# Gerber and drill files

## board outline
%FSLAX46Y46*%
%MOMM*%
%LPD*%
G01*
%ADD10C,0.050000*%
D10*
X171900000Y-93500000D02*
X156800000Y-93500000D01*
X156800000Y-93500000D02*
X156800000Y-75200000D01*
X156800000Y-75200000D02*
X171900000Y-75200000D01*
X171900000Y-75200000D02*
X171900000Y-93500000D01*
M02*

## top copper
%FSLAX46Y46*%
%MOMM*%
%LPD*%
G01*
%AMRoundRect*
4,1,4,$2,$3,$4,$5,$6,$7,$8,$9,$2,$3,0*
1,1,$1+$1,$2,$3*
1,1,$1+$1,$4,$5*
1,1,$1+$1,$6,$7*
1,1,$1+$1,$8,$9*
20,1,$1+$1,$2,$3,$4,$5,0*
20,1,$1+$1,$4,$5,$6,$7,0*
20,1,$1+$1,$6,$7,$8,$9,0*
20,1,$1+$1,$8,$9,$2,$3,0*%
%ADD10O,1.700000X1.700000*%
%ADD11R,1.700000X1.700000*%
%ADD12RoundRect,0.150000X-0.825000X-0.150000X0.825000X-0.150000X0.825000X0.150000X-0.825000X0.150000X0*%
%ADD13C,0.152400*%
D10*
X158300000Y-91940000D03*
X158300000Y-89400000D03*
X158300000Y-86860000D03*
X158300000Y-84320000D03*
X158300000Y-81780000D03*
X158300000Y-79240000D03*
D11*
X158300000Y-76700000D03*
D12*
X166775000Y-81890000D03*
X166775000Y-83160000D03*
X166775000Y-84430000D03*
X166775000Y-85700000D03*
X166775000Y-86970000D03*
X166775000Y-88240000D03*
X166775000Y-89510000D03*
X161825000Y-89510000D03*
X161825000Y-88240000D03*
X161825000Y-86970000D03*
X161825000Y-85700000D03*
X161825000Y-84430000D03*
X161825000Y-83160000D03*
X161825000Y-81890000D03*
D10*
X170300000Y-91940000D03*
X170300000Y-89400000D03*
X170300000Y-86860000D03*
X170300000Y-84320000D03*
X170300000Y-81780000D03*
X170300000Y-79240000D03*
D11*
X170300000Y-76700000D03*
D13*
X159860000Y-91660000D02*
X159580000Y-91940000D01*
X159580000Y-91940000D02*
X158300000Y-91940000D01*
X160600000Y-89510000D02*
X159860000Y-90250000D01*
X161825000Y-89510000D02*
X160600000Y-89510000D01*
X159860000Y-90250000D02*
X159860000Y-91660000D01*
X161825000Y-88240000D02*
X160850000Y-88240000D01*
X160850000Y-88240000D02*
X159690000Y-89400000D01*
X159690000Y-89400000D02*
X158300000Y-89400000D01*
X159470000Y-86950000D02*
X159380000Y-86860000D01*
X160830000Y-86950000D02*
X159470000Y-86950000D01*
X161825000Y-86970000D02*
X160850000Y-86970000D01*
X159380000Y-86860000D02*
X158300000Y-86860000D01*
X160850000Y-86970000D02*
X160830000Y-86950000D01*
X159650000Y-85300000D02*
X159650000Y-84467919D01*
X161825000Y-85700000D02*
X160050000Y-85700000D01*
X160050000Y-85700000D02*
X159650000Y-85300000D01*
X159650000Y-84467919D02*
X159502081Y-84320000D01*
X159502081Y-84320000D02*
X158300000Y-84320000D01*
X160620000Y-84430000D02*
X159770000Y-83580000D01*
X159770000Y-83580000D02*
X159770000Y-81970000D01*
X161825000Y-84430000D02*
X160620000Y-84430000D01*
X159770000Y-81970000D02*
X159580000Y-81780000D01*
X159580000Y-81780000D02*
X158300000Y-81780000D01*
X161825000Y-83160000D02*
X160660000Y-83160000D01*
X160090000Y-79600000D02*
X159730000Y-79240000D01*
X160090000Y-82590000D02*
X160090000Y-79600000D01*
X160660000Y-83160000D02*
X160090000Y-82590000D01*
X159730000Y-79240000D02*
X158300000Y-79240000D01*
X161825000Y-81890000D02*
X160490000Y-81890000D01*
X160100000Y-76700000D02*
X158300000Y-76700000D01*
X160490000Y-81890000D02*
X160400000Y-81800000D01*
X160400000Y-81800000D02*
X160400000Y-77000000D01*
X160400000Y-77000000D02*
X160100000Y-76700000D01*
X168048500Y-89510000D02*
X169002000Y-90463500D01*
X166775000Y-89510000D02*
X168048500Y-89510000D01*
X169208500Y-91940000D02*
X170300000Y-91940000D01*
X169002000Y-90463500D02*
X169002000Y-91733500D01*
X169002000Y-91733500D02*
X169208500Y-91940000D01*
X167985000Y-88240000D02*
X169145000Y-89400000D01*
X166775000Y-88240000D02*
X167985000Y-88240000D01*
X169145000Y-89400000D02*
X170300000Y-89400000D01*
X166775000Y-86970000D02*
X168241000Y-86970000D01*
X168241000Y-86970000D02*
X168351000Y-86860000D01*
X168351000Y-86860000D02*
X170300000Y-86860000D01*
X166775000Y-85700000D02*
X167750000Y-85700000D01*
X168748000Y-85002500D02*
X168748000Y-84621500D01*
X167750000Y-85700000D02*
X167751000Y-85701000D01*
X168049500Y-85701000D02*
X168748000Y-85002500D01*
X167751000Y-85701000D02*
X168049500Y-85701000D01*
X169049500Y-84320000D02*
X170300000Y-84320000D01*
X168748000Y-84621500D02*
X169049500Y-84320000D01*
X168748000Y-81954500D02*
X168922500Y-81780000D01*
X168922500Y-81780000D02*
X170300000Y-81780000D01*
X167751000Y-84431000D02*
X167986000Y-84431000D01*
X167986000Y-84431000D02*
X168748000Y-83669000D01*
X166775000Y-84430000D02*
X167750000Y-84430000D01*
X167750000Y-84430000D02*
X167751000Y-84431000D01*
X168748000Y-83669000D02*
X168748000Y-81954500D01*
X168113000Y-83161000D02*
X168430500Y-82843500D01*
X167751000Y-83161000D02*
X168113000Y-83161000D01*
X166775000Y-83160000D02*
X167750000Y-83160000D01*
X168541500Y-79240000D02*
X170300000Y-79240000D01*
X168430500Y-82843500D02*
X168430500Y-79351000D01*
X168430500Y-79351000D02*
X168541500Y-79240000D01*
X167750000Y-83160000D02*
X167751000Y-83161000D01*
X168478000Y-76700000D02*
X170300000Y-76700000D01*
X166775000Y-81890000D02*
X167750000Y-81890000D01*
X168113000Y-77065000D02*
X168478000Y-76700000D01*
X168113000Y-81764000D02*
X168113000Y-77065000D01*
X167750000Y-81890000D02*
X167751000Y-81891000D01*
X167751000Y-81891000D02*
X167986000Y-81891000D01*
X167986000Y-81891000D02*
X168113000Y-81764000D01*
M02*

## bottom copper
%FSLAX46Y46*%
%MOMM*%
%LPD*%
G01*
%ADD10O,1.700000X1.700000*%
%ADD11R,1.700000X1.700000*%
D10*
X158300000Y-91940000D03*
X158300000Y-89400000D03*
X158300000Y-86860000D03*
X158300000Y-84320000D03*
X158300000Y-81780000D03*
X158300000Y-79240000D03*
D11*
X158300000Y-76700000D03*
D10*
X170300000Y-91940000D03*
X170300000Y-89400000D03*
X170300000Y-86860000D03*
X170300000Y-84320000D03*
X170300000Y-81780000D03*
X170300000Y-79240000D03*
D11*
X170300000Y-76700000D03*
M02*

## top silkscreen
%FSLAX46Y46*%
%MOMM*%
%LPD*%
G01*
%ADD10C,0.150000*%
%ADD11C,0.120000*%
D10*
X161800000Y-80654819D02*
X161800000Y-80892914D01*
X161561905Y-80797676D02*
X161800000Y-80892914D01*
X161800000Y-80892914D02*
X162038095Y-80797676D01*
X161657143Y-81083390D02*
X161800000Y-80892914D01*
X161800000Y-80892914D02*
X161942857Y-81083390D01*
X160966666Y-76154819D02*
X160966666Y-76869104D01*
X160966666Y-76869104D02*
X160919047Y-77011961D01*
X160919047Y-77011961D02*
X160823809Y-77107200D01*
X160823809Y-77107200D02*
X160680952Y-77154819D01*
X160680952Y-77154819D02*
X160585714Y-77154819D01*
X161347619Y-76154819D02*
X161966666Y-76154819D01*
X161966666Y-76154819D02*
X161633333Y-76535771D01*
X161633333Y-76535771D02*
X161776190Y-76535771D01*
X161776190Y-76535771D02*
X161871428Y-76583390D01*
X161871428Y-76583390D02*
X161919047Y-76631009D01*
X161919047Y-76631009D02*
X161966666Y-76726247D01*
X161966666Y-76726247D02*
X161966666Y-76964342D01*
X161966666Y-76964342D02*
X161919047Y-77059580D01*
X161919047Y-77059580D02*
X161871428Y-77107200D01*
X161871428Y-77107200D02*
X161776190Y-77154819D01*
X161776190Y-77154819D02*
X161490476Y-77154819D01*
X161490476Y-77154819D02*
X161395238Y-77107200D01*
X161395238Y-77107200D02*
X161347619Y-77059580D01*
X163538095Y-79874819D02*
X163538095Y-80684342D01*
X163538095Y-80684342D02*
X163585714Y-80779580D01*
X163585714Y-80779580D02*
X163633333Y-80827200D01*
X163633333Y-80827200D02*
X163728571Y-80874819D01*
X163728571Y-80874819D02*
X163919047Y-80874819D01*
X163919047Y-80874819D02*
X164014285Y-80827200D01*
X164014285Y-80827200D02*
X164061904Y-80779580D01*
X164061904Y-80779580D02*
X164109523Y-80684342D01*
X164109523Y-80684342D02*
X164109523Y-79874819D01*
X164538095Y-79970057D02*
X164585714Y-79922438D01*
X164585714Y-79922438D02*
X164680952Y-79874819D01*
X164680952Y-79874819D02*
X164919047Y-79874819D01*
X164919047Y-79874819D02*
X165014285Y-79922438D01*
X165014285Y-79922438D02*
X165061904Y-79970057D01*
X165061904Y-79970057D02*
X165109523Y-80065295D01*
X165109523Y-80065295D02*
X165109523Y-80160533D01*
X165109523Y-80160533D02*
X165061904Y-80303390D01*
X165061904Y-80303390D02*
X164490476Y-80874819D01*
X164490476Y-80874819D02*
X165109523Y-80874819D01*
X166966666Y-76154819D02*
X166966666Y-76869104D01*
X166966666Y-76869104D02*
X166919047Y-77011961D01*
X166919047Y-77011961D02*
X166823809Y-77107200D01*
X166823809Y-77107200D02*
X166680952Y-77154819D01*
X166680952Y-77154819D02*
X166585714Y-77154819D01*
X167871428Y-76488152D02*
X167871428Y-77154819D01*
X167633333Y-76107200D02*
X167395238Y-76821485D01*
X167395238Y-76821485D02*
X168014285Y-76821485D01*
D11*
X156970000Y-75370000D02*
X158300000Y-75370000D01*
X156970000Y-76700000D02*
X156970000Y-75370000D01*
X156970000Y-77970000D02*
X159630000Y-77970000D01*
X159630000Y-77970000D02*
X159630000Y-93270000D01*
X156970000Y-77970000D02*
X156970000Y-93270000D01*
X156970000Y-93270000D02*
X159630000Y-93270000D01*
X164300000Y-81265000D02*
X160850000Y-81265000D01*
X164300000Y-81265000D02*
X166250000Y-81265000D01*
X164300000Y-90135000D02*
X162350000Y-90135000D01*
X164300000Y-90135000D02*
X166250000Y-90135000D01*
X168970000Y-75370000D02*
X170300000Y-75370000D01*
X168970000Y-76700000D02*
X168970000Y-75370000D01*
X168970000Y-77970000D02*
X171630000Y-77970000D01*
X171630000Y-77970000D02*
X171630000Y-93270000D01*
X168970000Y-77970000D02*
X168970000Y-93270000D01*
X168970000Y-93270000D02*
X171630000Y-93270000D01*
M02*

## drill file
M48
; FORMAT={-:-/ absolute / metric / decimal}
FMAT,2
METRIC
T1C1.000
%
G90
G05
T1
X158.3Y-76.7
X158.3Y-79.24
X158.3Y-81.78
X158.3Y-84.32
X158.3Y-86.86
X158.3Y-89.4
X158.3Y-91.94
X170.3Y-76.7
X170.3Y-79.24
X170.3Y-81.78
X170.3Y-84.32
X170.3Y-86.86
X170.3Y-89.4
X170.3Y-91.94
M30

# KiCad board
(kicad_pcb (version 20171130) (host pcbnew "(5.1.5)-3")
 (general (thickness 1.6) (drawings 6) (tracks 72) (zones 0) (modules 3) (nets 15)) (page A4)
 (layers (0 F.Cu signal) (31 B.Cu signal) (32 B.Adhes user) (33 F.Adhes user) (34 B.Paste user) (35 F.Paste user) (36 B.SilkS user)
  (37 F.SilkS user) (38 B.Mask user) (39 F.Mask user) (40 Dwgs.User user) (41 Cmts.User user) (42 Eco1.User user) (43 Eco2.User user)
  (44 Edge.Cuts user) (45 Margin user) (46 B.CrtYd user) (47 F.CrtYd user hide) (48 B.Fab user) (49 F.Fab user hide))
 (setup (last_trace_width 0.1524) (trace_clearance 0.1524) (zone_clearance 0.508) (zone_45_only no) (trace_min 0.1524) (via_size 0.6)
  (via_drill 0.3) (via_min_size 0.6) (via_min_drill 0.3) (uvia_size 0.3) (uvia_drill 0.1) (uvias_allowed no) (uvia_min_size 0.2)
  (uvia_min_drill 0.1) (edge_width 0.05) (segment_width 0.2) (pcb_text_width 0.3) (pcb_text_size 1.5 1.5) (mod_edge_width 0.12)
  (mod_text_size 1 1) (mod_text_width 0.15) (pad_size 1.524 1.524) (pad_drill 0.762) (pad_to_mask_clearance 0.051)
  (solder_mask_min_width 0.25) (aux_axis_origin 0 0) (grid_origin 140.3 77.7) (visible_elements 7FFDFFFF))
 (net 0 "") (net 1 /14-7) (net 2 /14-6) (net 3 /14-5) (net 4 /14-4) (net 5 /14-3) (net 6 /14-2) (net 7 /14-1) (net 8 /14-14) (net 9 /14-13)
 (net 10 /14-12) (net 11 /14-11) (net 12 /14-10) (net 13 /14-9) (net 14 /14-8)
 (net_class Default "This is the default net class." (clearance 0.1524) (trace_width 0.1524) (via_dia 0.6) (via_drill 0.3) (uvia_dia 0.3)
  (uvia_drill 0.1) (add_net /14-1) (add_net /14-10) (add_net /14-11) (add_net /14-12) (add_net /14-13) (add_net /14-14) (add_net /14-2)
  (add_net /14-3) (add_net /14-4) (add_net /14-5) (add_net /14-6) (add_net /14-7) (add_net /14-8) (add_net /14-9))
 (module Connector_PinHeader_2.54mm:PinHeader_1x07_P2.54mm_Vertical (layer F.Cu) (at 158.3 76.7)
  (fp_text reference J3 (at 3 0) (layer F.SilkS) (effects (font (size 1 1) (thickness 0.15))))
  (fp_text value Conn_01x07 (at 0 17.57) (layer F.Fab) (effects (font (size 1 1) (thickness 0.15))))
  (fp_line (start -1.33 -1.33) (end 0 -1.33) (layer F.SilkS) (width 0.12))
  (fp_line (start -1.33 0) (end -1.33 -1.33) (layer F.SilkS) (width 0.12))
  (fp_line (start -1.33 1.27) (end 1.33 1.27) (layer F.SilkS) (width 0.12))
  (fp_line (start 1.33 1.27) (end 1.33 16.57) (layer F.SilkS) (width 0.12))
  (fp_line (start -1.33 1.27) (end -1.33 16.57) (layer F.SilkS) (width 0.12))
  (fp_line (start -1.33 16.57) (end 1.33 16.57) (layer F.SilkS) (width 0.12))
  (pad 7 thru_hole oval (at 0 15.24) (size 1.7 1.7) (drill 1) (layers *.Cu *.Mask) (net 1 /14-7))
  (pad 6 thru_hole oval (at 0 12.7) (size 1.7 1.7) (drill 1) (layers *.Cu *.Mask) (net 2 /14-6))
  (pad 5 thru_hole oval (at 0 10.16) (size 1.7 1.7) (drill 1) (layers *.Cu *.Mask) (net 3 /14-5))
  (pad 4 thru_hole oval (at 0 7.62) (size 1.7 1.7) (drill 1) (layers *.Cu *.Mask) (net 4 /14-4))
  (pad 3 thru_hole oval (at 0 5.08) (size 1.7 1.7) (drill 1) (layers *.Cu *.Mask) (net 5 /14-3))
  (pad 2 thru_hole oval (at 0 2.54) (size 1.7 1.7) (drill 1) (layers *.Cu *.Mask) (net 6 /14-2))
  (pad 1 thru_hole rect (at 0 0) (size 1.7 1.7) (drill 1) (layers *.Cu *.Mask) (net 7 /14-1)))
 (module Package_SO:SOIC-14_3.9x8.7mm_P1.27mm (layer F.Cu) (at 164.3 85.7)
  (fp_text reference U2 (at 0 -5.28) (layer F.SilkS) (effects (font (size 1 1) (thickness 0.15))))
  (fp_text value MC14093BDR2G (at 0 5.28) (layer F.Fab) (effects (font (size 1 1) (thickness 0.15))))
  (fp_line (start 0 -4.435) (end -3.45 -4.435) (layer F.SilkS) (width 0.12))
  (fp_line (start 0 -4.435) (end 1.95 -4.435) (layer F.SilkS) (width 0.12))
  (fp_line (start 0 4.435) (end -1.95 4.435) (layer F.SilkS) (width 0.12))
  (fp_line (start 0 4.435) (end 1.95 4.435) (layer F.SilkS) (width 0.12))
  (pad 14 smd roundrect (at 2.475 -3.81) (size 1.95 0.6) (layers F.Cu F.Paste F.Mask) (roundrect_rratio 0.25) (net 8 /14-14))
  (pad 13 smd roundrect (at 2.475 -2.54) (size 1.95 0.6) (layers F.Cu F.Paste F.Mask) (roundrect_rratio 0.25) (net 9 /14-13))
  (pad 12 smd roundrect (at 2.475 -1.27) (size 1.95 0.6) (layers F.Cu F.Paste F.Mask) (roundrect_rratio 0.25) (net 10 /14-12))
  (pad 11 smd roundrect (at 2.475 0) (size 1.95 0.6) (layers F.Cu F.Paste F.Mask) (roundrect_rratio 0.25) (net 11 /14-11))
  (pad 10 smd roundrect (at 2.475 1.27) (size 1.95 0.6) (layers F.Cu F.Paste F.Mask) (roundrect_rratio 0.25) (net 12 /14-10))
  (pad 9 smd roundrect (at 2.475 2.54) (size 1.95 0.6) (layers F.Cu F.Paste F.Mask) (roundrect_rratio 0.25) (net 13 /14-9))
  (pad 8 smd roundrect (at 2.475 3.81) (size 1.95 0.6) (layers F.Cu F.Paste F.Mask) (roundrect_rratio 0.25) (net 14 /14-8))
  (pad 7 smd roundrect (at -2.475 3.81) (size 1.95 0.6) (layers F.Cu F.Paste F.Mask) (roundrect_rratio 0.25) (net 1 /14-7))
  (pad 6 smd roundrect (at -2.475 2.54) (size 1.95 0.6) (layers F.Cu F.Paste F.Mask) (roundrect_rratio 0.25) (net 2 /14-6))
  (pad 5 smd roundrect (at -2.475 1.27) (size 1.95 0.6) (layers F.Cu F.Paste F.Mask) (roundrect_rratio 0.25) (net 3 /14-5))
  (pad 4 smd roundrect (at -2.475 0) (size 1.95 0.6) (layers F.Cu F.Paste F.Mask) (roundrect_rratio 0.25) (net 4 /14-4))
  (pad 3 smd roundrect (at -2.475 -1.27) (size 1.95 0.6) (layers F.Cu F.Paste F.Mask) (roundrect_rratio 0.25) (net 5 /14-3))
  (pad 2 smd roundrect (at -2.475 -2.54) (size 1.95 0.6) (layers F.Cu F.Paste F.Mask) (roundrect_rratio 0.25) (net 6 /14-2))
  (pad 1 smd roundrect (at -2.475 -3.81) (size 1.95 0.6) (layers F.Cu F.Paste F.Mask) (roundrect_rratio 0.25) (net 7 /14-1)))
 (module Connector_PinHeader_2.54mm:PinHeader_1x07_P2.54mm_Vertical (layer F.Cu) (at 170.3 76.7)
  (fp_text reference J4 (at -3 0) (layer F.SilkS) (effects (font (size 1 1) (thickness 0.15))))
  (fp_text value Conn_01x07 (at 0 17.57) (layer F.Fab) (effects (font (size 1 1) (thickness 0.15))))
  (fp_line (start -1.33 -1.33) (end 0 -1.33) (layer F.SilkS) (width 0.12))
  (fp_line (start -1.33 0) (end -1.33 -1.33) (layer F.SilkS) (width 0.12))
  (fp_line (start -1.33 1.27) (end 1.33 1.27) (layer F.SilkS) (width 0.12))
  (fp_line (start 1.33 1.27) (end 1.33 16.57) (layer F.SilkS) (width 0.12))
  (fp_line (start -1.33 1.27) (end -1.33 16.57) (layer F.SilkS) (width 0.12))
  (fp_line (start -1.33 16.57) (end 1.33 16.57) (layer F.SilkS) (width 0.12))
  (pad 7 thru_hole oval (at 0 15.24) (size 1.7 1.7) (drill 1) (layers *.Cu *.Mask) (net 14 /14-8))
  (pad 6 thru_hole oval (at 0 12.7) (size 1.7 1.7) (drill 1) (layers *.Cu *.Mask) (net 13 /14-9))
  (pad 5 thru_hole oval (at 0 10.16) (size 1.7 1.7) (drill 1) (layers *.Cu *.Mask) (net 12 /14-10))
  (pad 4 thru_hole oval (at 0 7.62) (size 1.7 1.7) (drill 1) (layers *.Cu *.Mask) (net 11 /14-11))
  (pad 3 thru_hole oval (at 0 5.08) (size 1.7 1.7) (drill 1) (layers *.Cu *.Mask) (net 10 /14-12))
  (pad 2 thru_hole oval (at 0 2.54) (size 1.7 1.7) (drill 1) (layers *.Cu *.Mask) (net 9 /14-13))
  (pad 1 thru_hole rect (at 0 0) (size 1.7 1.7) (drill 1) (layers *.Cu *.Mask) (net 8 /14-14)))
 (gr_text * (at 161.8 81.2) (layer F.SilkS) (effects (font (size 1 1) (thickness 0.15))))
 (gr_line (start 171.9 93.5) (end 156.8 93.5) (layer Edge.Cuts) (width 0.05))
 (gr_line (start 156.8 93.5) (end 156.8 75.2) (layer Edge.Cuts) (width 0.05))
 (gr_line (start 156.8 75.2) (end 171.9 75.2) (layer Edge.Cuts) (width 0.05))
 (gr_line (start 171.9 75.2) (end 171.9 93.5) (layer Edge.Cuts) (width 0.05))
 (segment (start 159.86 91.66) (end 159.58 91.94) (width 0.1524) (layer F.Cu) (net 1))
 (segment (start 159.58 91.94) (end 158.3 91.94) (width 0.1524) (layer F.Cu) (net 1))
 (segment (start 160.6 89.51) (end 159.86 90.25) (width 0.1524) (layer F.Cu) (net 1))
 (segment (start 161.825 89.51) (end 160.6 89.51) (width 0.1524) (layer F.Cu) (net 1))
 (segment (start 159.86 90.25) (end 159.86 91.66) (width 0.1524) (layer F.Cu) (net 1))
 (segment (start 161.825 88.24) (end 160.85 88.24) (width 0.1524) (layer F.Cu) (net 2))
 (segment (start 160.85 88.24) (end 159.69 89.4) (width 0.1524) (layer F.Cu) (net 2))
 (segment (start 159.69 89.4) (end 158.3 89.4) (width 0.1524) (layer F.Cu) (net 2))
 (segment (start 159.47 86.95) (end 159.38 86.86) (width 0.1524) (layer F.Cu) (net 3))
 (segment (start 160.83 86.95) (end 159.47 86.95) (width 0.1524) (layer F.Cu) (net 3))
 (segment (start 161.825 86.97) (end 160.85 86.97) (width 0.1524) (layer F.Cu) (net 3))
 (segment (start 159.38 86.86) (end 158.3 86.86) (width 0.1524) (layer F.Cu) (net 3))
 (segment (start 160.85 86.97) (end 160.83 86.95) (width 0.1524) (layer F.Cu) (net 3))
 (segment (start 159.65 85.3) (end 159.65 84.467919) (width 0.1524) (layer F.Cu) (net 4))
 (segment (start 161.825 85.7) (end 160.05 85.7) (width 0.1524) (layer F.Cu) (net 4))
 (segment (start 160.05 85.7) (end 159.65 85.3) (width 0.1524) (layer F.Cu) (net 4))
 (segment (start 159.65 84.467919) (end 159.502081 84.32) (width 0.1524) (layer F.Cu) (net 4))
 (segment (start 159.502081 84.32) (end 158.3 84.32) (width 0.1524) (layer F.Cu) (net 4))
 (segment (start 160.62 84.43) (end 159.77 83.58) (width 0.1524) (layer F.Cu) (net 5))
 (segment (start 159.77 83.58) (end 159.77 81.97) (width 0.1524) (layer F.Cu) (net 5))
 (segment (start 161.825 84.43) (end 160.62 84.43) (width 0.1524) (layer F.Cu) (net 5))
 (segment (start 159.77 81.97) (end 159.58 81.78) (width 0.1524) (layer F.Cu) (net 5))
 (segment (start 159.58 81.78) (end 158.3 81.78) (width 0.1524) (layer F.Cu) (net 5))
 (segment (start 161.825 83.16) (end 160.66 83.16) (width 0.1524) (layer F.Cu) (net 6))
 (segment (start 160.09 79.6) (end 159.73 79.24) (width 0.1524) (layer F.Cu) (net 6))
 (segment (start 160.09 82.59) (end 160.09 79.6) (width 0.1524) (layer F.Cu) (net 6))
 (segment (start 160.66 83.16) (end 160.09 82.59) (width 0.1524) (layer F.Cu) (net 6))
 (segment (start 159.73 79.24) (end 158.3 79.24) (width 0.1524) (layer F.Cu) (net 6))
 (segment (start 161.825 81.89) (end 160.49 81.89) (width 0.1524) (layer F.Cu) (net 7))
 (segment (start 160.1 76.7) (end 158.3 76.7) (width 0.1524) (layer F.Cu) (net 7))
 (segment (start 160.49 81.89) (end 160.4 81.8) (width 0.1524) (layer F.Cu) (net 7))
 (segment (start 160.4 81.8) (end 160.4 77) (width 0.1524) (layer F.Cu) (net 7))
 (segment (start 160.4 77) (end 160.1 76.7) (width 0.1524) (layer F.Cu) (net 7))
 (segment (start 168.0485 89.51) (end 169.002 90.4635) (width 0.1524) (layer F.Cu) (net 14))
 (segment (start 166.775 89.51) (end 168.0485 89.51) (width 0.1524) (layer F.Cu) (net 14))
 (segment (start 169.2085 91.94) (end 170.3 91.94) (width 0.1524) (layer F.Cu) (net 14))
 (segment (start 169.002 90.4635) (end 169.002 91.7335) (width 0.1524) (layer F.Cu) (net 14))
 (segment (start 169.002 91.7335) (end 169.2085 91.94) (width 0.1524) (layer F.Cu) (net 14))
 (segment (start 167.985 88.24) (end 169.145 89.4) (width 0.1524) (layer F.Cu) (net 13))
 (segment (start 166.775 88.24) (end 167.985 88.24) (width 0.1524) (layer F.Cu) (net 13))
 (segment (start 169.145 89.4) (end 170.3 89.4) (width 0.1524) (layer F.Cu) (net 13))
 (segment (start 166.775 86.97) (end 168.241 86.97) (width 0.1524) (layer F.Cu) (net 12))
 (segment (start 168.241 86.97) (end 168.351 86.86) (width 0.1524) (layer F.Cu) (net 12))
 (segment (start 168.351 86.86) (end 170.3 86.86) (width 0.1524) (layer F.Cu) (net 12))
 (segment (start 166.775 85.7) (end 167.75 85.7) (width 0.1524) (layer F.Cu) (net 11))
 (segment (start 168.748 85.0025) (end 168.748 84.6215) (width 0.1524) (layer F.Cu) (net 11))
 (segment (start 167.75 85.7) (end 167.751 85.701) (width 0.1524) (layer F.Cu) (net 11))
 (segment (start 168.0495 85.701) (end 168.748 85.0025) (width 0.1524) (layer F.Cu) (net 11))
 (segment (start 167.751 85.701) (end 168.0495 85.701) (width 0.1524) (layer F.Cu) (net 11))
 (segment (start 169.0495 84.32) (end 170.3 84.32) (width 0.1524) (layer F.Cu) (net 11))
 (segment (start 168.748 84.6215) (end 169.0495 84.32) (width 0.1524) (layer F.Cu) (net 11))
 (segment (start 168.748 81.9545) (end 168.9225 81.78) (width 0.1524) (layer F.Cu) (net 10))
 (segment (start 168.9225 81.78) (end 170.3 81.78) (width 0.1524) (layer F.Cu) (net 10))
 (segment (start 167.751 84.431) (end 167.986 84.431) (width 0.1524) (layer F.Cu) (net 10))
 (segment (start 167.986 84.431) (end 168.748 83.669) (width 0.1524) (layer F.Cu) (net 10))
 (segment (start 166.775 84.43) (end 167.75 84.43) (width 0.1524) (layer F.Cu) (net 10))
 (segment (start 167.75 84.43) (end 167.751 84.431) (width 0.1524) (layer F.Cu) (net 10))
 (segment (start 168.748 83.669) (end 168.748 81.9545) (width 0.1524) (layer F.Cu) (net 10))
 (segment (start 168.113 83.161) (end 168.4305 82.8435) (width 0.1524) (layer F.Cu) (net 9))
 (segment (start 167.751 83.161) (end 168.113 83.161) (width 0.1524) (layer F.Cu) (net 9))
 (segment (start 166.775 83.16) (end 167.75 83.16) (width 0.1524) (layer F.Cu) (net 9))
 (segment (start 168.5415 79.24) (end 170.3 79.24) (width 0.1524) (layer F.Cu) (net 9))
 (segment (start 168.4305 82.8435) (end 168.4305 79.351) (width 0.1524) (layer F.Cu) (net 9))
 (segment (start 168.4305 79.351) (end 168.5415 79.24) (width 0.1524) (layer F.Cu) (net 9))
 (segment (start 167.75 83.16) (end 167.751 83.161) (width 0.1524) (layer F.Cu) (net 9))
 (segment (start 168.478 76.7) (end 170.3 76.7) (width 0.1524) (layer F.Cu) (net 8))
 (segment (start 166.775 81.89) (end 167.75 81.89) (width 0.1524) (layer F.Cu) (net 8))
 (segment (start 168.113 77.065) (end 168.478 76.7) (width 0.1524) (layer F.Cu) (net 8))
 (segment (start 168.113 81.764) (end 168.113 77.065) (width 0.1524) (layer F.Cu) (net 8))
 (segment (start 167.75 81.89) (end 167.751 81.891) (width 0.1524) (layer F.Cu) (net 8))
 (segment (start 167.751 81.891) (end 167.986 81.891) (width 0.1524) (layer F.Cu) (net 8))
 (segment (start 167.986 81.891) (end 168.113 81.764) (width 0.1524) (layer F.Cu) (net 8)))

